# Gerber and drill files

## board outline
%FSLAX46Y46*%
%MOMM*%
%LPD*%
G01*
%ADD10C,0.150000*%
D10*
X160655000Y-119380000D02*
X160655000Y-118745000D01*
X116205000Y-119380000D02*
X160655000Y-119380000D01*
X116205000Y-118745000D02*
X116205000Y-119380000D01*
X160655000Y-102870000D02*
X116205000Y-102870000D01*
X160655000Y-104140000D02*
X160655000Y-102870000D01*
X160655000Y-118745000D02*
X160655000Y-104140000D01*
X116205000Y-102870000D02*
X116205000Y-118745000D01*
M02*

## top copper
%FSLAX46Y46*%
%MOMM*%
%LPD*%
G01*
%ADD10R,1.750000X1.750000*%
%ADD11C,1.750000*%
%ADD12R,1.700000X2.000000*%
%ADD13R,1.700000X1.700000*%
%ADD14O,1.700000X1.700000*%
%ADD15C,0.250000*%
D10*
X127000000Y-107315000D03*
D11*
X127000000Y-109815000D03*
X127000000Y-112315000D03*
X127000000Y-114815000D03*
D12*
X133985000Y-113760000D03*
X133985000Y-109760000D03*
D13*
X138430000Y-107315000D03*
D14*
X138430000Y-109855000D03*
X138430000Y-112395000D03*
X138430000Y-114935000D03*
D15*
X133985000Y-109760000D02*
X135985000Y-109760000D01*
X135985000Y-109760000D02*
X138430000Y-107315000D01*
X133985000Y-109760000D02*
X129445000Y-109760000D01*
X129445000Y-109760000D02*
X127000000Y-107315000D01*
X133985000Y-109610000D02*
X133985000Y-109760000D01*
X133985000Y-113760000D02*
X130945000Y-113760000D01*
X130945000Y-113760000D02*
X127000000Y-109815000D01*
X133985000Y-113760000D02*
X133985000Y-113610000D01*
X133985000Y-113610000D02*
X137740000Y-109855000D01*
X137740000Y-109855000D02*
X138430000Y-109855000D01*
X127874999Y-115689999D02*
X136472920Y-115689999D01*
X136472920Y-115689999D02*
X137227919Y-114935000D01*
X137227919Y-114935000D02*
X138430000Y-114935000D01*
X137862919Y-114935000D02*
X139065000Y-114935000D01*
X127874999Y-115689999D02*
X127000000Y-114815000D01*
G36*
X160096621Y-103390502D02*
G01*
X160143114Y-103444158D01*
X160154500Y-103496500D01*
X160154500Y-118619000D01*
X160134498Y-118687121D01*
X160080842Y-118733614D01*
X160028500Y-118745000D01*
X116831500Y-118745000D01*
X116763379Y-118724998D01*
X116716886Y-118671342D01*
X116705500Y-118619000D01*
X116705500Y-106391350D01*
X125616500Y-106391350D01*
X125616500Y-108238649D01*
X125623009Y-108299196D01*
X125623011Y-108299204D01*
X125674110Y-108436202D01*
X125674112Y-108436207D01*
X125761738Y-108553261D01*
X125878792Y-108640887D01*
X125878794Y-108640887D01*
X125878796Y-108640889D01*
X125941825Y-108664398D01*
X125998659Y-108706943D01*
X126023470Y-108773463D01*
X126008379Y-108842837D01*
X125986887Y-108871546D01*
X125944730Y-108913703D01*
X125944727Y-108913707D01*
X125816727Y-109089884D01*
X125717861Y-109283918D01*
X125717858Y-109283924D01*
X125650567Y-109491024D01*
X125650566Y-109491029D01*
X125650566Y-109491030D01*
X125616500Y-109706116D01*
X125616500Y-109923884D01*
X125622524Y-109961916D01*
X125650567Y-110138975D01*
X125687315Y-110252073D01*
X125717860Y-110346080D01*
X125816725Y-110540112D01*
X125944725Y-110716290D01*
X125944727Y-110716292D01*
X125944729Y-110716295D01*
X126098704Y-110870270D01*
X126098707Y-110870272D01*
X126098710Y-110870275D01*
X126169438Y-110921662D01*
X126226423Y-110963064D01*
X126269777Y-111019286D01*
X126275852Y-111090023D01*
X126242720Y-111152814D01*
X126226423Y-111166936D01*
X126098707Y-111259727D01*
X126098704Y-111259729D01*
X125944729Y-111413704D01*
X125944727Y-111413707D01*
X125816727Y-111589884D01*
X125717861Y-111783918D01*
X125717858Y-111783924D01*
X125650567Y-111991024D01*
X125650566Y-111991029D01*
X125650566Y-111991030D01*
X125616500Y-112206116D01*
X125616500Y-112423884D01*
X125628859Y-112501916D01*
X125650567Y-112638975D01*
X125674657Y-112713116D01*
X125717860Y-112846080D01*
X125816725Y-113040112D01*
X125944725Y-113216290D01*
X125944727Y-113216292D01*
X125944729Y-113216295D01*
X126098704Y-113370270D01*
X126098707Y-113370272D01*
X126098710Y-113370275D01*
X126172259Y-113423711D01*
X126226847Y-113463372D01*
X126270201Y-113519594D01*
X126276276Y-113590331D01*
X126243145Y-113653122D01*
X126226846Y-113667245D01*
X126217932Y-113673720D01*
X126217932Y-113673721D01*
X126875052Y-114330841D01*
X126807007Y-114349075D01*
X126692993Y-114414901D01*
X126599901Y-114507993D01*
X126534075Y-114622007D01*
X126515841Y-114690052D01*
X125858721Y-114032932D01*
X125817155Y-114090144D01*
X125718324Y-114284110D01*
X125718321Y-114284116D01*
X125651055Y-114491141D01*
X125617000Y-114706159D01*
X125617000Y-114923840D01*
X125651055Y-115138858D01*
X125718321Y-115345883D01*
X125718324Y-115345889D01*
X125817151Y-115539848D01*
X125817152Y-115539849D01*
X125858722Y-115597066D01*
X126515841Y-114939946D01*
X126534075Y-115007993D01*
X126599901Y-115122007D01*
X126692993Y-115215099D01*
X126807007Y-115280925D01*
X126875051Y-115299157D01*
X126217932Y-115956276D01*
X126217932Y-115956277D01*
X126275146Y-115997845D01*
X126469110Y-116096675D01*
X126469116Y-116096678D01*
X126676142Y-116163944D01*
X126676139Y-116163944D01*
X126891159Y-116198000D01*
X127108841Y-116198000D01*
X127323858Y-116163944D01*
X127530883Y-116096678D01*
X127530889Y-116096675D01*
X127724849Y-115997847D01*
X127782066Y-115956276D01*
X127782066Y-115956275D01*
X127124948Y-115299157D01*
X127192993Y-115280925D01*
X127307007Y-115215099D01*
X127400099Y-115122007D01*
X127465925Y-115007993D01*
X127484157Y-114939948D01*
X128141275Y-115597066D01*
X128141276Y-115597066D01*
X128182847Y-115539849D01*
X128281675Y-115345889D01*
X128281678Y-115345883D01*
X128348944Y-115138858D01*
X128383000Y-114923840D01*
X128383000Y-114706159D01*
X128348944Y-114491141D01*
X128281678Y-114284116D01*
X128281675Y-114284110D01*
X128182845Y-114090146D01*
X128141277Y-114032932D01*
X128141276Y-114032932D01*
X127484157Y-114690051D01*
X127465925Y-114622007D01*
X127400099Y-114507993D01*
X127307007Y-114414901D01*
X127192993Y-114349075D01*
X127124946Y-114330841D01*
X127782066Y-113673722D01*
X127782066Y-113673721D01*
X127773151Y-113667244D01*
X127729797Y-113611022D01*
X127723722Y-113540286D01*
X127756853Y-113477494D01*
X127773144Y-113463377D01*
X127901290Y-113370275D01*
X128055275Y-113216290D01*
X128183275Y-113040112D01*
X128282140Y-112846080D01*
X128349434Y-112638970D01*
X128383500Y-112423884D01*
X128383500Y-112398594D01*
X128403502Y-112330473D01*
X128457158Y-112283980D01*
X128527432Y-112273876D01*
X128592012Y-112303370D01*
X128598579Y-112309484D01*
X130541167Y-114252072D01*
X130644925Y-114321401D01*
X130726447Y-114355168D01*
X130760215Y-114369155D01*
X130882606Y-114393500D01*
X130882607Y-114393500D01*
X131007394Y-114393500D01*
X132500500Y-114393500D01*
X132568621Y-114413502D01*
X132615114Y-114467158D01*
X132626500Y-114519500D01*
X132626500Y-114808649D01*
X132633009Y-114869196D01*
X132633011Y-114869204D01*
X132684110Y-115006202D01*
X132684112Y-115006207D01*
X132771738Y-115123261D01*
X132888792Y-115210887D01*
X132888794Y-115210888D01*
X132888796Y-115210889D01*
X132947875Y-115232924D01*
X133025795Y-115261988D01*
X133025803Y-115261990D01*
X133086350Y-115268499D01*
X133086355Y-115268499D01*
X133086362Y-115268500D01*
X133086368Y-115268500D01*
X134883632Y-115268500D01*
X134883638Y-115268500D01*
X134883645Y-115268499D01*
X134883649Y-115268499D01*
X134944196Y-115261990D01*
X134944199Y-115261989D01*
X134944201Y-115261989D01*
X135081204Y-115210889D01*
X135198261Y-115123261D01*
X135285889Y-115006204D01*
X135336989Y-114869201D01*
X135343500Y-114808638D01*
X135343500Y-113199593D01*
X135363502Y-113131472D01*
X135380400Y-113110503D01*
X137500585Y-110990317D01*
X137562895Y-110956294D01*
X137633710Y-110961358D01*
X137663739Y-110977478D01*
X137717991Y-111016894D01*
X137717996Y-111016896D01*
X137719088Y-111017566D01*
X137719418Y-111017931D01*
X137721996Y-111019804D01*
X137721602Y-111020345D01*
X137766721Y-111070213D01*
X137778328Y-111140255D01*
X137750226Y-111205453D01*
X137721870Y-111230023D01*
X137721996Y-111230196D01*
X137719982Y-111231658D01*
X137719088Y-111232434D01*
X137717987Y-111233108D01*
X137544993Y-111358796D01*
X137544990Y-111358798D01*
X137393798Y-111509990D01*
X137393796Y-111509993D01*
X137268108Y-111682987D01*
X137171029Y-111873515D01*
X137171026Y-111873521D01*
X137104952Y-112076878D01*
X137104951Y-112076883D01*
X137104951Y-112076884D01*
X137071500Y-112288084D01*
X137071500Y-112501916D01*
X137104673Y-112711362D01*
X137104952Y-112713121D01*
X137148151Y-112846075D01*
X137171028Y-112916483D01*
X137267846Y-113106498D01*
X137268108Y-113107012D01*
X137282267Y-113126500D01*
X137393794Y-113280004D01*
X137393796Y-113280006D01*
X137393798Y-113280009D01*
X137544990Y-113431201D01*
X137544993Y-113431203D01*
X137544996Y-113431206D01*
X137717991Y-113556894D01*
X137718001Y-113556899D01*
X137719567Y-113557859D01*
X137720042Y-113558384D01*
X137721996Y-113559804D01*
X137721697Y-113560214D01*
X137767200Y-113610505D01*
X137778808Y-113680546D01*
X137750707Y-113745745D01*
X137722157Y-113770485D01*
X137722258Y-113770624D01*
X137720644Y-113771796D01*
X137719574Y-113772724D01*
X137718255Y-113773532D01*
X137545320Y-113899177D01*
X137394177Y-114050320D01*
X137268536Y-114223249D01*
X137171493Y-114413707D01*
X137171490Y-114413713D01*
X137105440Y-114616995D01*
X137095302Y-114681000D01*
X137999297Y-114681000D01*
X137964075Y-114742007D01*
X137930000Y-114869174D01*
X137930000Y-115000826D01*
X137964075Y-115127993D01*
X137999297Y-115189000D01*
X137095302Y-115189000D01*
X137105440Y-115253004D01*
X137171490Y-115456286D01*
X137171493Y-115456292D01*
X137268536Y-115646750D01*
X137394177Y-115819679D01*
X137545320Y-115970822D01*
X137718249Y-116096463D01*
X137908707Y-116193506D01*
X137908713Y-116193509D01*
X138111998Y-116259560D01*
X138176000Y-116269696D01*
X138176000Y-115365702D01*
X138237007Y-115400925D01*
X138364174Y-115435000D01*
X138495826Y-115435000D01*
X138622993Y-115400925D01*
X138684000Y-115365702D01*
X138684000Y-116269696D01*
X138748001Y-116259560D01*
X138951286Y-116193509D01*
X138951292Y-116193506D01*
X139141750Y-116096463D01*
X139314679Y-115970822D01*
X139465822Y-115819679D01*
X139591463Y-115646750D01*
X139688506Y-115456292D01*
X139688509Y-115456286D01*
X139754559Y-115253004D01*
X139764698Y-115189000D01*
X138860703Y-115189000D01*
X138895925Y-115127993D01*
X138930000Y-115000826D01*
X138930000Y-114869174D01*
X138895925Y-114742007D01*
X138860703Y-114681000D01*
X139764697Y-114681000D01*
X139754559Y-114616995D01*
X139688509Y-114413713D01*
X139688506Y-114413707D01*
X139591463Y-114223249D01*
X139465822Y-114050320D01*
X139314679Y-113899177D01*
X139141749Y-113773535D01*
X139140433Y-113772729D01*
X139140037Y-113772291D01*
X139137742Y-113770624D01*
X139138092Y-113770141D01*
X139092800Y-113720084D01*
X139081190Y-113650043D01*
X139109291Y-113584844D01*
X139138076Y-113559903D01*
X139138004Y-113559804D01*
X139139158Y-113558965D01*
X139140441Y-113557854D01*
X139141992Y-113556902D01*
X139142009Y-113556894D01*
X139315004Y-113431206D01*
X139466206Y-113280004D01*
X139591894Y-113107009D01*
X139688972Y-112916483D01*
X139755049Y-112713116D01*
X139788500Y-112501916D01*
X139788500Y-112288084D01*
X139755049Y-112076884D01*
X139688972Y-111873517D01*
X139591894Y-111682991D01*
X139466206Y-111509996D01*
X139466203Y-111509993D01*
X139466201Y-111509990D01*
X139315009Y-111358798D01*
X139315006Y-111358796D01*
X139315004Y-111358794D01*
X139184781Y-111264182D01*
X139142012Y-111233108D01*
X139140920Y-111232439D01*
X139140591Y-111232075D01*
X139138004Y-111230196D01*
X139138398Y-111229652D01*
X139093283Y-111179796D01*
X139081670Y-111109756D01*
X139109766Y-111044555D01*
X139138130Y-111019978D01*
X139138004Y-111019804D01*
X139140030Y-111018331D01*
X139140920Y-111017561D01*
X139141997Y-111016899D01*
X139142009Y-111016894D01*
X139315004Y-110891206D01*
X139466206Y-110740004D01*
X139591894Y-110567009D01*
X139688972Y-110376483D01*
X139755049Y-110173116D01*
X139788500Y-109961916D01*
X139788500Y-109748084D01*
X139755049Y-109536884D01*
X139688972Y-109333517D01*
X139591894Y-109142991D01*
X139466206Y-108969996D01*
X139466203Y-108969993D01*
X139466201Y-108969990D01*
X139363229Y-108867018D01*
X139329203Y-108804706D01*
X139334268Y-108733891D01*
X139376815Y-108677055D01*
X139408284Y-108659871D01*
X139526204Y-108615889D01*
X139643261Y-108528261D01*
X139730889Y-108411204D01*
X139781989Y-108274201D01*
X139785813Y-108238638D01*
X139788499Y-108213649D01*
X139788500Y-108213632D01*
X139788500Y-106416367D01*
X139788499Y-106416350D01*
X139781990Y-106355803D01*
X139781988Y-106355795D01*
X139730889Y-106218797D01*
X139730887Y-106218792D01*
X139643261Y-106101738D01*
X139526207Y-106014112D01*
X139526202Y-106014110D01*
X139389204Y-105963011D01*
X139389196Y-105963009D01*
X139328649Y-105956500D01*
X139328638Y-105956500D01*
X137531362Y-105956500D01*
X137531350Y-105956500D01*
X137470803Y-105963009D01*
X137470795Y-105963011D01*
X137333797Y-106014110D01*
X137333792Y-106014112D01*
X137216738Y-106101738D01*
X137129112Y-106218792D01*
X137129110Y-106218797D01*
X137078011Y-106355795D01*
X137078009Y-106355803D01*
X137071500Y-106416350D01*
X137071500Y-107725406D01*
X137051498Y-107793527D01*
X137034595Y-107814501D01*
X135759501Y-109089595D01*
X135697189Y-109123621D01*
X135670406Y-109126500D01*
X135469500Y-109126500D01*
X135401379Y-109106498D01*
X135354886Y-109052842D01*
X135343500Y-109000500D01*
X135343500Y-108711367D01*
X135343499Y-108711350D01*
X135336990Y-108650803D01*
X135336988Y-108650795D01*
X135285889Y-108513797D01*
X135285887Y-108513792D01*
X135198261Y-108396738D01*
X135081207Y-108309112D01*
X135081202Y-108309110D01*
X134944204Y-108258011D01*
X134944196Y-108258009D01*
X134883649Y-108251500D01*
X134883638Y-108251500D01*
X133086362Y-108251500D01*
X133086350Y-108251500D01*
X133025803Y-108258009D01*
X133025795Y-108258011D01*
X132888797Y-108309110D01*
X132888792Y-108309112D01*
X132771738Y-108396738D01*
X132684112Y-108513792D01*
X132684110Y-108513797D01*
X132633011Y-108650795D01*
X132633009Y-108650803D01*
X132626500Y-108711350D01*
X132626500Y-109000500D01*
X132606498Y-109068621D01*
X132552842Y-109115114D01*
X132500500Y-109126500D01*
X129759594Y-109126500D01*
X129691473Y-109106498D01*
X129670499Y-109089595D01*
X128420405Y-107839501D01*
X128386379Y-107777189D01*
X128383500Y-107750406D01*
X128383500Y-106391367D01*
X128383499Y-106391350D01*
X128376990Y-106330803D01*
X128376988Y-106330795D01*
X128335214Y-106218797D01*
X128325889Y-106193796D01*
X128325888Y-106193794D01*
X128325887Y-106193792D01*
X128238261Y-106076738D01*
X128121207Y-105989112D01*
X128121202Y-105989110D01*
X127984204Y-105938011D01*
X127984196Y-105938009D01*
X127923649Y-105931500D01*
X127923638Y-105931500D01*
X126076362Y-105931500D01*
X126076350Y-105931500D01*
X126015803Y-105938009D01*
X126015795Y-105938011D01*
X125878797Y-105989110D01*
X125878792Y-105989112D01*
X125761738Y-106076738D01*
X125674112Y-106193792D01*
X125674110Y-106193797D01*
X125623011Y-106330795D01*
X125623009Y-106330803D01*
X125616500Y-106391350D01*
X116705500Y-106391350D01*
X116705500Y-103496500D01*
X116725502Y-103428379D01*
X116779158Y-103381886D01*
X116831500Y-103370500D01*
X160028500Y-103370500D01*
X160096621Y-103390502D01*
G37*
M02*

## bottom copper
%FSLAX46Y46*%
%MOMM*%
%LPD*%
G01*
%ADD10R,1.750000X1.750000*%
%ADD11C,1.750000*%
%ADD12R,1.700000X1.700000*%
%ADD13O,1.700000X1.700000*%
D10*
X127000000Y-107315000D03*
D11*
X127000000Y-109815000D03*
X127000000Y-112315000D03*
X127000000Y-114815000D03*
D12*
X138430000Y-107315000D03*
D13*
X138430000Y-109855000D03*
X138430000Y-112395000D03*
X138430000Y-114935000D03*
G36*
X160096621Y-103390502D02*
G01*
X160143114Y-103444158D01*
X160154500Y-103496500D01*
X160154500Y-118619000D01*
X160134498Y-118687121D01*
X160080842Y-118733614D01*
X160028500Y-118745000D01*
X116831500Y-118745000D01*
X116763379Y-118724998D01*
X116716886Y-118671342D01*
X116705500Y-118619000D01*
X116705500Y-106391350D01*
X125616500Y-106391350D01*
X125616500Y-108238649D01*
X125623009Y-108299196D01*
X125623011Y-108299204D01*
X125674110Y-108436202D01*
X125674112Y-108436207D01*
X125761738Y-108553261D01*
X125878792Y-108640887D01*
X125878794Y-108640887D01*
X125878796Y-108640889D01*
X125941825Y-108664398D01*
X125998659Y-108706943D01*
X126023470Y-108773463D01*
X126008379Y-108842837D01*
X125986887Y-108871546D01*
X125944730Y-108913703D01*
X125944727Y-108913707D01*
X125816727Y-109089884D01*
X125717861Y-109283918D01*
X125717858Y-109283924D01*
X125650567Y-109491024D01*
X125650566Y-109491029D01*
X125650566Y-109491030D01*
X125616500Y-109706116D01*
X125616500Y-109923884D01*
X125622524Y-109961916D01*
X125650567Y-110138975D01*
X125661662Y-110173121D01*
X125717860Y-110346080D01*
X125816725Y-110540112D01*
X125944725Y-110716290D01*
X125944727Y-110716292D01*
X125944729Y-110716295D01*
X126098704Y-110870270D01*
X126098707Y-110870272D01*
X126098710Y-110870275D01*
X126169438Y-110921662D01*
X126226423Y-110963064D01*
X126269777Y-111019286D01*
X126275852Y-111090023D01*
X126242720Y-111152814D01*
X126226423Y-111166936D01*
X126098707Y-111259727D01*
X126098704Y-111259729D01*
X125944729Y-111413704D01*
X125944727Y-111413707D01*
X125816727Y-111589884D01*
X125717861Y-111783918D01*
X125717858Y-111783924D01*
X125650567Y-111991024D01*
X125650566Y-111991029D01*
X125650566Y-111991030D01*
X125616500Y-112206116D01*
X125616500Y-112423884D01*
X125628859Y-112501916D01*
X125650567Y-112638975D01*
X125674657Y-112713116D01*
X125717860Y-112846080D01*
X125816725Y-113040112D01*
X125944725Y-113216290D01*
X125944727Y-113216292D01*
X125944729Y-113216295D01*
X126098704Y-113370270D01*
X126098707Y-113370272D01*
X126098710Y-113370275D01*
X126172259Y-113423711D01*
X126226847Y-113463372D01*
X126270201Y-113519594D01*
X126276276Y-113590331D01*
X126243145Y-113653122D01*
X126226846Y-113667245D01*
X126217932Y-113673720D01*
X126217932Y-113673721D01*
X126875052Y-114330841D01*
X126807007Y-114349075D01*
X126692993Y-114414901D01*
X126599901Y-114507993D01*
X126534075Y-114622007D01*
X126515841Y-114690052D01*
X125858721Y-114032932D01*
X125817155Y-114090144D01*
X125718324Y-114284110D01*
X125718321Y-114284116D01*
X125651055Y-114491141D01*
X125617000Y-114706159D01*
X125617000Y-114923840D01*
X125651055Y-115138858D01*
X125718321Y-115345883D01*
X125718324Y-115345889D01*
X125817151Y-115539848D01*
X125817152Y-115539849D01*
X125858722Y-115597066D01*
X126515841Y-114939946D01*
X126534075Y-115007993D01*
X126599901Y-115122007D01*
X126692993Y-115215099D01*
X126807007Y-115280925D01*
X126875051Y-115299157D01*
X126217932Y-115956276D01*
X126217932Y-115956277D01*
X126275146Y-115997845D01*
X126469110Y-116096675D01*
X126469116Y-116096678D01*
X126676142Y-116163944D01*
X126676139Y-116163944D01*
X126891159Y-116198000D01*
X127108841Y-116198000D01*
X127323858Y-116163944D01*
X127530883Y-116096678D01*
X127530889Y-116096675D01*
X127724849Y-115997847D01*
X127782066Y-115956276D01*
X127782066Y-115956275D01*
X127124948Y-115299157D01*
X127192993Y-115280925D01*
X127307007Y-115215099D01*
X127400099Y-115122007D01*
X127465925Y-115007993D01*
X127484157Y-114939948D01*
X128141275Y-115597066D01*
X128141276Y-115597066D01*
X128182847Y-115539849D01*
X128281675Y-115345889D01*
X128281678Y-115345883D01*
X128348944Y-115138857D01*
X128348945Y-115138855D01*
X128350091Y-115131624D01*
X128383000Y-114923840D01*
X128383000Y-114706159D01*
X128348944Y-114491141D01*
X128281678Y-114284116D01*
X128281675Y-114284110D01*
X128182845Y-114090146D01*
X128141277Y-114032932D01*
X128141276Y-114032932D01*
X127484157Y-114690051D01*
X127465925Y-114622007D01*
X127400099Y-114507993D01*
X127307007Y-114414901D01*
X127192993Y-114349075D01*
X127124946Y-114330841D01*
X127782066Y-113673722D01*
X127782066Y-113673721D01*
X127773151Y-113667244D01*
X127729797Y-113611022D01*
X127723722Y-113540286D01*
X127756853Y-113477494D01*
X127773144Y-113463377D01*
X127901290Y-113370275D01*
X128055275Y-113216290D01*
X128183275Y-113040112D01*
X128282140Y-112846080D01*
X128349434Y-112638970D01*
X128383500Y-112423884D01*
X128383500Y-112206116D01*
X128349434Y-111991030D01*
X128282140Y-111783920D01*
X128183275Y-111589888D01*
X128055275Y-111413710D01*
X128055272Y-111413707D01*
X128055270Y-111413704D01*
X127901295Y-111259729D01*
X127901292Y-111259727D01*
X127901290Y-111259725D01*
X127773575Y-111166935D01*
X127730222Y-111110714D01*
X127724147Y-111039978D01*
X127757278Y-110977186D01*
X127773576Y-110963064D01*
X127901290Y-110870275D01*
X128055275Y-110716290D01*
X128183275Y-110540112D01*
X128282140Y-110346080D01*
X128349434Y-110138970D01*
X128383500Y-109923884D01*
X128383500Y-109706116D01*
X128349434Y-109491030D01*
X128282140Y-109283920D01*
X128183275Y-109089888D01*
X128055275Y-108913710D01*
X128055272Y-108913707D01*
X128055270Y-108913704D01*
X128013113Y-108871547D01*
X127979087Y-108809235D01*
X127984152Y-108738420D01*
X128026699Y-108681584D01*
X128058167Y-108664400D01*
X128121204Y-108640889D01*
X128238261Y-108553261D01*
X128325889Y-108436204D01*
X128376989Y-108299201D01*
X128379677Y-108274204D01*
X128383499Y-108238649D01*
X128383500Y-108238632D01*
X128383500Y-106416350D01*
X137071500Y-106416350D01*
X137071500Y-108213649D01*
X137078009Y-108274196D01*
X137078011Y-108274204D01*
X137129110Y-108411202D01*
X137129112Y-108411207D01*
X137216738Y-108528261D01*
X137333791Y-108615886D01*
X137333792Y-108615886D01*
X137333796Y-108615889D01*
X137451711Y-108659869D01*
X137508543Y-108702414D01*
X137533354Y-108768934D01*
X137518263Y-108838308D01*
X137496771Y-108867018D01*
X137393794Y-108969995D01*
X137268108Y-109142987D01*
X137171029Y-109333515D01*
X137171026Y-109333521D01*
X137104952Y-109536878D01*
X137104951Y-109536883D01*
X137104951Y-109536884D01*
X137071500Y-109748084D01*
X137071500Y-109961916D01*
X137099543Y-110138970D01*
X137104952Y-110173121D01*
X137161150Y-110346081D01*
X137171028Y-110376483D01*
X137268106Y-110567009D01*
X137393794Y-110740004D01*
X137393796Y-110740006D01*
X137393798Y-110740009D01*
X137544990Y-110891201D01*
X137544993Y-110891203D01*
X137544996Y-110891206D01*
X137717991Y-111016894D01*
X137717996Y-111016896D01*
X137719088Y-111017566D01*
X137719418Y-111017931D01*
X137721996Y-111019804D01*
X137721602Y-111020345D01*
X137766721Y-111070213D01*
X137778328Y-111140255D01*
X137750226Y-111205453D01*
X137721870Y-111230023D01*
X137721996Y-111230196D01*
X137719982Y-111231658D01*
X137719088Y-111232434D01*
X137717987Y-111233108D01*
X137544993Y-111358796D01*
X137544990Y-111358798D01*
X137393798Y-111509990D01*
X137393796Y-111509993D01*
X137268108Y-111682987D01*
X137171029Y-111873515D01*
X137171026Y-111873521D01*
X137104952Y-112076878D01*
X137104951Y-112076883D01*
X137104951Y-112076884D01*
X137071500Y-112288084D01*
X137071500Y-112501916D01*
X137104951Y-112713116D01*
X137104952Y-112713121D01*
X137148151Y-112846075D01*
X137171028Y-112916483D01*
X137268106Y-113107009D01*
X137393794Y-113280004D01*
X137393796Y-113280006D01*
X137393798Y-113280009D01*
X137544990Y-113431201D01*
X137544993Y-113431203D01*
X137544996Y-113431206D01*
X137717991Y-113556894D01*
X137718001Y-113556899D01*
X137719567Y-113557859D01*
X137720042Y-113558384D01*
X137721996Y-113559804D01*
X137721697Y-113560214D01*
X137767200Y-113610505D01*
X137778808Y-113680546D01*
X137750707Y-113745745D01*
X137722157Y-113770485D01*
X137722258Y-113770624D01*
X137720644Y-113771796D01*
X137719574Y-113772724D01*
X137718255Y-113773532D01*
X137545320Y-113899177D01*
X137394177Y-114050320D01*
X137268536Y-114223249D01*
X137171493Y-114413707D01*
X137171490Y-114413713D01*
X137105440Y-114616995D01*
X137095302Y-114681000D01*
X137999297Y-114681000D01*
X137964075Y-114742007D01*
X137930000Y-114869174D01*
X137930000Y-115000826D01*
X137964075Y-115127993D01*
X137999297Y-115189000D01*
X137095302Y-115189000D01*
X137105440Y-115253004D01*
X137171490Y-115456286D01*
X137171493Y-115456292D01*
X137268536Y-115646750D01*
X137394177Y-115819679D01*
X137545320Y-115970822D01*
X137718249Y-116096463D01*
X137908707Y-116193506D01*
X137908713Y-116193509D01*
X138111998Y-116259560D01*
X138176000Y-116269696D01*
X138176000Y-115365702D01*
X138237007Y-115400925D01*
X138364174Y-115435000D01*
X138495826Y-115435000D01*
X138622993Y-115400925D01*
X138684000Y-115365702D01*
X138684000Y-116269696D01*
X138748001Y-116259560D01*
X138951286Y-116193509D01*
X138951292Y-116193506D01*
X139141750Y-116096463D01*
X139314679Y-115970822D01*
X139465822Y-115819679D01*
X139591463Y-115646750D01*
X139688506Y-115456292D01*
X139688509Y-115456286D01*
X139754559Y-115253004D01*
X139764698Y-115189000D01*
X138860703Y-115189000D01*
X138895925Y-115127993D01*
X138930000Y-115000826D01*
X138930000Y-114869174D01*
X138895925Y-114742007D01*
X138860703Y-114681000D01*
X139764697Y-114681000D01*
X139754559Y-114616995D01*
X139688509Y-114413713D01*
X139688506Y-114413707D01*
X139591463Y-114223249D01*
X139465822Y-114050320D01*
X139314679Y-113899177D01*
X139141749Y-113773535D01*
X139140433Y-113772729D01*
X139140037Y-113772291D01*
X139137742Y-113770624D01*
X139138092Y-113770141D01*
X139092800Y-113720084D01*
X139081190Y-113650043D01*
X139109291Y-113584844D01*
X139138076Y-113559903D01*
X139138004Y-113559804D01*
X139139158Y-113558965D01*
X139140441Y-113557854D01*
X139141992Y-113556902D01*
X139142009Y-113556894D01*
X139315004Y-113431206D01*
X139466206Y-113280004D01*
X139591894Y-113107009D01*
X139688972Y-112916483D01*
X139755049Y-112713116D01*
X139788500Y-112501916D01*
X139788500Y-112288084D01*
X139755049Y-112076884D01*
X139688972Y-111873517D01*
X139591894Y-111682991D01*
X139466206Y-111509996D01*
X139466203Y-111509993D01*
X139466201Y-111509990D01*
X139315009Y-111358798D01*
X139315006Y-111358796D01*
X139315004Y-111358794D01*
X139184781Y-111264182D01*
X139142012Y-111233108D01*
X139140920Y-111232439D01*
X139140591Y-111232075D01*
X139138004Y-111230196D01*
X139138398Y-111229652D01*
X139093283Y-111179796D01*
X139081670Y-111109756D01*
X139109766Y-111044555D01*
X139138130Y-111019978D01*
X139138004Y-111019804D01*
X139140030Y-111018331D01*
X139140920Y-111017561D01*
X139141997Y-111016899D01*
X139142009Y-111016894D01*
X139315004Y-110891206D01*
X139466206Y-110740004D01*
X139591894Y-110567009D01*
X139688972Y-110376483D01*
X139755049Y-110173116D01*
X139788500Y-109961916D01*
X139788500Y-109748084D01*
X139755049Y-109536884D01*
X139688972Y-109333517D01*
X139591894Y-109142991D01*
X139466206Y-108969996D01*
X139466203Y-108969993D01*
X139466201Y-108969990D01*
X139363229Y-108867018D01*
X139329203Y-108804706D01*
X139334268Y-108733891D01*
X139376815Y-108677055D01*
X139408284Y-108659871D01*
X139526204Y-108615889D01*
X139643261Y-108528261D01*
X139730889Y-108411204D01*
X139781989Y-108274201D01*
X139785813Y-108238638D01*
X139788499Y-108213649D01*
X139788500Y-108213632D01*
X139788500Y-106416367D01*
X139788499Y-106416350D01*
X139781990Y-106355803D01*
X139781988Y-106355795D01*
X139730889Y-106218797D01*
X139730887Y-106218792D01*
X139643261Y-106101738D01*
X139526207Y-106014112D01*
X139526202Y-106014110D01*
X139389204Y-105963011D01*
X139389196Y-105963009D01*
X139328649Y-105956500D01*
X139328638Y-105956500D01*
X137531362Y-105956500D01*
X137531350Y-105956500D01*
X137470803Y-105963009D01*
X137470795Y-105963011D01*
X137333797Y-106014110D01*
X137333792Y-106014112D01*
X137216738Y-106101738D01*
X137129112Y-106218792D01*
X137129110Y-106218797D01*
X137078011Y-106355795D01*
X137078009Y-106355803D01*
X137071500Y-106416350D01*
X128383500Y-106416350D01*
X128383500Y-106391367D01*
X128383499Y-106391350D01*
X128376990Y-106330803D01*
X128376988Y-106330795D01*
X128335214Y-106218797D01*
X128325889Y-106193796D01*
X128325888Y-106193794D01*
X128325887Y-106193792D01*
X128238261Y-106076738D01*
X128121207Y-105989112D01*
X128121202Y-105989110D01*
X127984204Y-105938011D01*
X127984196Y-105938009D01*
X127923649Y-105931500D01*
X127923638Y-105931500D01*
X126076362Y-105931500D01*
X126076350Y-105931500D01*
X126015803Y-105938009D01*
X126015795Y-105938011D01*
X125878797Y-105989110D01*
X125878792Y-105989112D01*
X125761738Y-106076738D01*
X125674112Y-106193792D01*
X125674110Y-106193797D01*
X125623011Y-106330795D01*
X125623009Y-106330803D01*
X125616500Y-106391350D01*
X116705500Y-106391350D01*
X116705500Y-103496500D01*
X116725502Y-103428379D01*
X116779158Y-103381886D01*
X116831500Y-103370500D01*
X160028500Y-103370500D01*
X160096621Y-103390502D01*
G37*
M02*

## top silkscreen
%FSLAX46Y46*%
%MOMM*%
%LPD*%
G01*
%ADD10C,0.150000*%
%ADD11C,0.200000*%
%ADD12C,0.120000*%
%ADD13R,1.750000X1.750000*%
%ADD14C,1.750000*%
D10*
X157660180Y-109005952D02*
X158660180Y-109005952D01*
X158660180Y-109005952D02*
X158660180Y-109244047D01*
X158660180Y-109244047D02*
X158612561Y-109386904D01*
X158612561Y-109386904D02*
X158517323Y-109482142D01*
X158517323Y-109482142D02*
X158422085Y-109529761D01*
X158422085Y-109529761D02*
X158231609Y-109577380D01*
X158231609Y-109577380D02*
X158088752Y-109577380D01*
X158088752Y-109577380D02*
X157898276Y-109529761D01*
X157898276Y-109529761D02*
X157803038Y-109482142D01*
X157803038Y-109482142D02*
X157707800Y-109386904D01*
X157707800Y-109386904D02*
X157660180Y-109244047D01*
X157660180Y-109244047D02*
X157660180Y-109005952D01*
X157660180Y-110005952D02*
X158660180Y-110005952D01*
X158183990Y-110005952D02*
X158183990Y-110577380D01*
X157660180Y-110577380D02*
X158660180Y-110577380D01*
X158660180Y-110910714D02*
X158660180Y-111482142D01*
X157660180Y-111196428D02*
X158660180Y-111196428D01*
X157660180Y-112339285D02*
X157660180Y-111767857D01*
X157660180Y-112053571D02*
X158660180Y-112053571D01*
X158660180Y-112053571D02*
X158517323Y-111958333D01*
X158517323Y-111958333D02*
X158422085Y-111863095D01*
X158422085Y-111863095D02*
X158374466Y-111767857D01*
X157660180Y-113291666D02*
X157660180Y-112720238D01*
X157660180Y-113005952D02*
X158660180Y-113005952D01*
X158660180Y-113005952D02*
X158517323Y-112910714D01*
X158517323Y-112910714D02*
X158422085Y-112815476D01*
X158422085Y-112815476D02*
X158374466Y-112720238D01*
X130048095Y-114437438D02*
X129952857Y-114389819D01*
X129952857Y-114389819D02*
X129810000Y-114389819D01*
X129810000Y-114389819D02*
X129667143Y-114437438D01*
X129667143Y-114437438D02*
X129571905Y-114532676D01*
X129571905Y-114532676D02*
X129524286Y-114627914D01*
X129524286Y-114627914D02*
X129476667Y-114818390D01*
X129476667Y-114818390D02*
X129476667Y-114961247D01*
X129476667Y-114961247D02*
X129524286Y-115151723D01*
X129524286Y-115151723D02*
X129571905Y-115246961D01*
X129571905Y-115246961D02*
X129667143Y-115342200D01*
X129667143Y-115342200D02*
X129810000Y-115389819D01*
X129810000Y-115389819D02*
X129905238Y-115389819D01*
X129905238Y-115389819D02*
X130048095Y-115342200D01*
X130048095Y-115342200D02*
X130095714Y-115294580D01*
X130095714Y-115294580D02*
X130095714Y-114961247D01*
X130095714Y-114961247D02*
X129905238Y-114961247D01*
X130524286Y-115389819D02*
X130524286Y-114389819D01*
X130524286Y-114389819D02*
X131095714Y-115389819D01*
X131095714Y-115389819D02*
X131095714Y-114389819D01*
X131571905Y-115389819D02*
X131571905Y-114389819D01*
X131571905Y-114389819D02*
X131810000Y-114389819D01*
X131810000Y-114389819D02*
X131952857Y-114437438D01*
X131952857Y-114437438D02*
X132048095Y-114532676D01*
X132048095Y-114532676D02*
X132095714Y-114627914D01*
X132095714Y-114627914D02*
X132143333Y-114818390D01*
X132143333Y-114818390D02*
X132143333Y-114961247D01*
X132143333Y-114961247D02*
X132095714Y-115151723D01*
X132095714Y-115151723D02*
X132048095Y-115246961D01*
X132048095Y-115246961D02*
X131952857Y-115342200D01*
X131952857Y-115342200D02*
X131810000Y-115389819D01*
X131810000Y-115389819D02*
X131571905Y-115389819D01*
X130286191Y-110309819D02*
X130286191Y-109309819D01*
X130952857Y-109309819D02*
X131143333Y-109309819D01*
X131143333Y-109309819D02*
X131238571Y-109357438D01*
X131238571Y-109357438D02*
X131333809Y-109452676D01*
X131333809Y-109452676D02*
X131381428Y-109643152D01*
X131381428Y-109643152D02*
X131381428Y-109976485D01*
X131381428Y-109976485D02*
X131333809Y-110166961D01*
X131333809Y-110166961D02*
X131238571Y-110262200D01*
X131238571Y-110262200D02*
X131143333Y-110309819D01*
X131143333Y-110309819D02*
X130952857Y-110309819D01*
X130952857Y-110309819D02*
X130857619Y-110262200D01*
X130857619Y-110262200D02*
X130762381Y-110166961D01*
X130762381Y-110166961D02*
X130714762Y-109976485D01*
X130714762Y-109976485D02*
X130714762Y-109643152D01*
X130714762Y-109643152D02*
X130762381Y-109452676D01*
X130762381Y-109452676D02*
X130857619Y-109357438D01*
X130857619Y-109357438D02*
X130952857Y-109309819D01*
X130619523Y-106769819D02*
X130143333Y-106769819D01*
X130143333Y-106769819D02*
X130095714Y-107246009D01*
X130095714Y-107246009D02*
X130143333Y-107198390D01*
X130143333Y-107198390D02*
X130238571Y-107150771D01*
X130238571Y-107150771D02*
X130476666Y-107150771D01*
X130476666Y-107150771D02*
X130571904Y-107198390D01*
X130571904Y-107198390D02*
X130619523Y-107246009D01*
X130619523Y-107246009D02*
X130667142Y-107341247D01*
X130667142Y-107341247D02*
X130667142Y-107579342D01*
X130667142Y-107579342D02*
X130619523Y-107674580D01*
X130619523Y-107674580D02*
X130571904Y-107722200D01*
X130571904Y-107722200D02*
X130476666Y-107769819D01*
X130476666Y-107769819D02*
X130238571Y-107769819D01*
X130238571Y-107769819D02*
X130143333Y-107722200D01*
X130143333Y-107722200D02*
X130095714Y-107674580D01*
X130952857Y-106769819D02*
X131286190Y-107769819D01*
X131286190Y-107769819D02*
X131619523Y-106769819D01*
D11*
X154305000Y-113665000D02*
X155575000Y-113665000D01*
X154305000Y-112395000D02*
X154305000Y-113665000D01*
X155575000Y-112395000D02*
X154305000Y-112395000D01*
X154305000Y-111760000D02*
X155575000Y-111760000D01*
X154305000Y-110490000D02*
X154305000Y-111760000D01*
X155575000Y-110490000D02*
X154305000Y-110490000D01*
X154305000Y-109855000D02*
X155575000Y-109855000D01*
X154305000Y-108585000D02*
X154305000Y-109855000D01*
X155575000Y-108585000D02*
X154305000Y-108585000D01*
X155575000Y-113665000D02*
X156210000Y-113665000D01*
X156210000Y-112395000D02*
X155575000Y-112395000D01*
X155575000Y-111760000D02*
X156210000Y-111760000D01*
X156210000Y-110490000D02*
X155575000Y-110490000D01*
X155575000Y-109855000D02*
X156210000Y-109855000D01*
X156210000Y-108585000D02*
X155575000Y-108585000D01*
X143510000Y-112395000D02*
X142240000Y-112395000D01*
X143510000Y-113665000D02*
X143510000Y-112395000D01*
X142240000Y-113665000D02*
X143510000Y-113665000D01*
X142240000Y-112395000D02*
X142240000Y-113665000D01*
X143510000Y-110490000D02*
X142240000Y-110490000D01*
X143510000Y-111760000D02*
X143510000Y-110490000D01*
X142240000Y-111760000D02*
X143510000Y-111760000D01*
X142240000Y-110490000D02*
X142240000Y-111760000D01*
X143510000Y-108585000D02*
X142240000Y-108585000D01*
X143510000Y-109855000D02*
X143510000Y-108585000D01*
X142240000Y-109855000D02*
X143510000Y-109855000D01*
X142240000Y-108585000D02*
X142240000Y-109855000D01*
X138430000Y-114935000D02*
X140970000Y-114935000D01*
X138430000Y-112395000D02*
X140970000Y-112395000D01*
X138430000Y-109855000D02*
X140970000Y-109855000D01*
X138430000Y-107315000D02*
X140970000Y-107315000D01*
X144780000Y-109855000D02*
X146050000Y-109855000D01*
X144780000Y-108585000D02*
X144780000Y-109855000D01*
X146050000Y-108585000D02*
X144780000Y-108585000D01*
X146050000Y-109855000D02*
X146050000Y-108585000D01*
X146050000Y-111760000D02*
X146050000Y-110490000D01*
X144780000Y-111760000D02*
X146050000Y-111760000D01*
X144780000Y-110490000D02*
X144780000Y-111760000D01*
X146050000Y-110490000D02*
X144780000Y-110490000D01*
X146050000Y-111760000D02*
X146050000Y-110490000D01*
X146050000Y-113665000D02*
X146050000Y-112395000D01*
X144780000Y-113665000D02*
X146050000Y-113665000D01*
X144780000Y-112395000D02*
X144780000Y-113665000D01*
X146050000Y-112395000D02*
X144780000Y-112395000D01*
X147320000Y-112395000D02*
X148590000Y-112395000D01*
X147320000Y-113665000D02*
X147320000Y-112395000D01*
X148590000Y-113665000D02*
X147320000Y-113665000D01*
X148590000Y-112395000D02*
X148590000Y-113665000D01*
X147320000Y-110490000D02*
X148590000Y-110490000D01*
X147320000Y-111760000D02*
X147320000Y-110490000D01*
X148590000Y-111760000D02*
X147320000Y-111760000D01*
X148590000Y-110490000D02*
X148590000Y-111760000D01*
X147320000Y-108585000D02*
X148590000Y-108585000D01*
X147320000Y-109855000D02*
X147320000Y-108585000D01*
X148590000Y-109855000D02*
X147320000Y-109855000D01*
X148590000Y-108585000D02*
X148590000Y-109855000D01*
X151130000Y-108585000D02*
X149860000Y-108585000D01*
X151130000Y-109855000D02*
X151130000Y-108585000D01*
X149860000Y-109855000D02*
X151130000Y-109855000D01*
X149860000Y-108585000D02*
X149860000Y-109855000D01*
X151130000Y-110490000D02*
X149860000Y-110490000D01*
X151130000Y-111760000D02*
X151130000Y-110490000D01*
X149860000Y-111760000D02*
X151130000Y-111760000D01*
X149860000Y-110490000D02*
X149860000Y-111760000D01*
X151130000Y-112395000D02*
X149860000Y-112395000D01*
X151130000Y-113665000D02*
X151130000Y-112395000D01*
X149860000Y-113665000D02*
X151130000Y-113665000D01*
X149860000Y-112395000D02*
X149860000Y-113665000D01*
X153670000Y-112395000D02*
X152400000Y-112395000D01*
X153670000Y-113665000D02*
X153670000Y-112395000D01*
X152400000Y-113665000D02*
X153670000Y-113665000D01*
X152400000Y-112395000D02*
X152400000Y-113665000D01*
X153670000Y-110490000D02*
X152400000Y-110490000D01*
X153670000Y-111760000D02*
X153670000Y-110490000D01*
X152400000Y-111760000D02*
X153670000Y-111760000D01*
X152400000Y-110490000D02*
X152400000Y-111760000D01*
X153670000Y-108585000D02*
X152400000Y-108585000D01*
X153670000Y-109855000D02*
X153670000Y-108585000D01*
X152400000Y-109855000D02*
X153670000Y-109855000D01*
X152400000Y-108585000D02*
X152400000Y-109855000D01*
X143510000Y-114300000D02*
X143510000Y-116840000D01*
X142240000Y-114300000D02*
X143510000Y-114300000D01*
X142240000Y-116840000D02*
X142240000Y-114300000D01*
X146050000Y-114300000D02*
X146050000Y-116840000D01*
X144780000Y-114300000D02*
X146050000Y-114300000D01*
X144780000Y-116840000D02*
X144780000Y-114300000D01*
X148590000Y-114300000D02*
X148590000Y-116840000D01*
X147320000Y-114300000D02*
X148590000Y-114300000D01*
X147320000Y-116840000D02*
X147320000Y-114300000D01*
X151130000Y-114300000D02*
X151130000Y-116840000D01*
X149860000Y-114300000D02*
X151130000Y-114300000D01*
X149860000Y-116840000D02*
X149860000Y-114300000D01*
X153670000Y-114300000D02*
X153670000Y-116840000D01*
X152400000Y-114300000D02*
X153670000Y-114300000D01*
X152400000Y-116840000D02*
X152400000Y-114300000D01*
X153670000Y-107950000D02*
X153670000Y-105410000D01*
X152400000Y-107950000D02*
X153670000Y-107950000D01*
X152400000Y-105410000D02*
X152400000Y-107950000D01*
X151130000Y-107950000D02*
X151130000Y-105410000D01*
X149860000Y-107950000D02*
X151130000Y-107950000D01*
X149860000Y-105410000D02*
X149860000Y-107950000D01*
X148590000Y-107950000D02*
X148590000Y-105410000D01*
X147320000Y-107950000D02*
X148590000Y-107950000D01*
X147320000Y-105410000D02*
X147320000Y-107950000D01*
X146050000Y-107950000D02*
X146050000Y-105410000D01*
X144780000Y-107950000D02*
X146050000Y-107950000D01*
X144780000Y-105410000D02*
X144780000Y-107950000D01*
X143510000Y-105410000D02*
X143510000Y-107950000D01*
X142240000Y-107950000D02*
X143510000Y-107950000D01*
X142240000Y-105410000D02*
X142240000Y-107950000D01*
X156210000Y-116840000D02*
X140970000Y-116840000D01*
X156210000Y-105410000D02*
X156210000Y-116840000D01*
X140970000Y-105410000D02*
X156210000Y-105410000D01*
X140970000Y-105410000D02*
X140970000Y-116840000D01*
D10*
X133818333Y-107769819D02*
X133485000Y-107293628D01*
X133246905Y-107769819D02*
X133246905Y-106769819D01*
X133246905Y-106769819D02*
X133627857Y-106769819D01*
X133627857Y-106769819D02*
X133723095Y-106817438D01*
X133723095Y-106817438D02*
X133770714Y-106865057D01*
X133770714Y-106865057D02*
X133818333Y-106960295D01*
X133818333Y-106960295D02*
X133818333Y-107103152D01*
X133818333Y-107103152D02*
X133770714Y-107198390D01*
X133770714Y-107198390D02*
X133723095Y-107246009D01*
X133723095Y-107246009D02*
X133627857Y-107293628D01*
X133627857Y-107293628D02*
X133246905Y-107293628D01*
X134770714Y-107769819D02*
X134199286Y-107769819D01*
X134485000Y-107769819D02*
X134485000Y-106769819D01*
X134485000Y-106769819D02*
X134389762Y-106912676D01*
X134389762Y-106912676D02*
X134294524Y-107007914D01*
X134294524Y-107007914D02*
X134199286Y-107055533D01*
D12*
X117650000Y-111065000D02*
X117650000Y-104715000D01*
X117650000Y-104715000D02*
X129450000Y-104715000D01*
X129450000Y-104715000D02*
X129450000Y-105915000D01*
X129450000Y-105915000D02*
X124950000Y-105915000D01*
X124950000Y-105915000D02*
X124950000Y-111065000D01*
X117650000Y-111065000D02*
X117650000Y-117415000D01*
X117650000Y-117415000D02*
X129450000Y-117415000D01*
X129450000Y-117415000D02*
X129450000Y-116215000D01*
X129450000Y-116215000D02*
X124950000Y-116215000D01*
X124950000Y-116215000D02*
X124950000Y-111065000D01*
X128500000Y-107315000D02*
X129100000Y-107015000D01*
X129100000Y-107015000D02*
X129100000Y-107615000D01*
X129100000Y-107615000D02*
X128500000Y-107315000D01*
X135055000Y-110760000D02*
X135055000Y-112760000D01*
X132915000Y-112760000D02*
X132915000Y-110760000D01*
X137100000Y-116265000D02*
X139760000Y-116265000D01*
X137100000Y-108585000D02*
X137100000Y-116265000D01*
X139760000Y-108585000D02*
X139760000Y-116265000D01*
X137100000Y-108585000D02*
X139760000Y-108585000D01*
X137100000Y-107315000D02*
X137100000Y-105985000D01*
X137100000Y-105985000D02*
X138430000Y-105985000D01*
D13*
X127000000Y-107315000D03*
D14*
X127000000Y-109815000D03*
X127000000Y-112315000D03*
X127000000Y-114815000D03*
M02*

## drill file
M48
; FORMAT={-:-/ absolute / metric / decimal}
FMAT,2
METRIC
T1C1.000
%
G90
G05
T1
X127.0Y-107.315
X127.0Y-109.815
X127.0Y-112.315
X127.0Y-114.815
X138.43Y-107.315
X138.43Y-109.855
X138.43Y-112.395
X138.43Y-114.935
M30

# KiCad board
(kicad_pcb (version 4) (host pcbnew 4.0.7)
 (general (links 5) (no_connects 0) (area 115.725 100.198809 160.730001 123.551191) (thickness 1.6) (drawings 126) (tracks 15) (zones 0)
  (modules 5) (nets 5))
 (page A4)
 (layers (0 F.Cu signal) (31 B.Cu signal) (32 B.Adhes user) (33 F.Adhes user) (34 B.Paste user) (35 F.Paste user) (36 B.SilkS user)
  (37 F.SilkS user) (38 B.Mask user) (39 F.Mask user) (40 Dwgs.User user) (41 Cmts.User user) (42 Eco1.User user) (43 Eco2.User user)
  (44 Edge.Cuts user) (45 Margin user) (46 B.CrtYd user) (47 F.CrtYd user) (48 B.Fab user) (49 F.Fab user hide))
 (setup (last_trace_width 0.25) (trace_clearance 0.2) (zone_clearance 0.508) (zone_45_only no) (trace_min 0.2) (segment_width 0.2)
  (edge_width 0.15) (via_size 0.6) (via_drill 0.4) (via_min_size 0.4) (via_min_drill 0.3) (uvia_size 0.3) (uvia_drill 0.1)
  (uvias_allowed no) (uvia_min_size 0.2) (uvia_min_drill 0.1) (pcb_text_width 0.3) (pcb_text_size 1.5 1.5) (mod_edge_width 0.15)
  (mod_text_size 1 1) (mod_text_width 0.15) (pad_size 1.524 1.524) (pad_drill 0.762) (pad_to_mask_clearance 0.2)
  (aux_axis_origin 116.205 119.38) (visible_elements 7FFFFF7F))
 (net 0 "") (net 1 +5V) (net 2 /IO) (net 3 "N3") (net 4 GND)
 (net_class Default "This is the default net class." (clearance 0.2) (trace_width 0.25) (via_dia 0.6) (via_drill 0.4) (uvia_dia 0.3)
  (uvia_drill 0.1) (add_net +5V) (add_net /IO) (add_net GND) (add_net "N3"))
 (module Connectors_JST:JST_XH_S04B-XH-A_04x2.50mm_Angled (layer F.Cu) (at 127 107.315 270)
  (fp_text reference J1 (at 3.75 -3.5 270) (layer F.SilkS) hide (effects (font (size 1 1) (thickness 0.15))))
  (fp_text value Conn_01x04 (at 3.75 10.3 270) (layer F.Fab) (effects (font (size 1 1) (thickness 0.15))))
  (fp_line (start 3.75 9.35) (end -2.6 9.35) (layer F.SilkS) (width 0.12))
  (fp_line (start -2.6 9.35) (end -2.6 -2.45) (layer F.SilkS) (width 0.12))
  (fp_line (start -2.6 -2.45) (end -1.4 -2.45) (layer F.SilkS) (width 0.12))
  (fp_line (start -1.4 -2.45) (end -1.4 2.05) (layer F.SilkS) (width 0.12))
  (fp_line (start -1.4 2.05) (end 3.75 2.05) (layer F.SilkS) (width 0.12))
  (fp_line (start 3.75 9.35) (end 10.1 9.35) (layer F.SilkS) (width 0.12))
  (fp_line (start 10.1 9.35) (end 10.1 -2.45) (layer F.SilkS) (width 0.12))
  (fp_line (start 10.1 -2.45) (end 8.9 -2.45) (layer F.SilkS) (width 0.12))
  (fp_line (start 8.9 -2.45) (end 8.9 2.05) (layer F.SilkS) (width 0.12))
  (fp_line (start 8.9 2.05) (end 3.75 2.05) (layer F.SilkS) (width 0.12))
  (fp_line (start 0 -1.5) (end -0.3 -2.1) (layer F.SilkS) (width 0.12))
  (fp_line (start -0.3 -2.1) (end 0.3 -2.1) (layer F.SilkS) (width 0.12))
  (fp_line (start 0.3 -2.1) (end 0 -1.5) (layer F.SilkS) (width 0.12))
  (pad 1 thru_hole rect (at 0 0 270) (size 1.75 1.75) (drill 1) (layers *.Cu *.Mask F.SilkS) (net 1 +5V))
  (pad 2 thru_hole circle (at 2.5 0 270) (size 1.75 1.75) (drill 1) (layers *.Cu *.Mask F.SilkS) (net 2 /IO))
  (pad 3 thru_hole circle (at 5 0 270) (size 1.75 1.75) (drill 1) (layers *.Cu *.Mask F.SilkS) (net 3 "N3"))
  (pad 4 thru_hole circle (at 7.5 0 270) (size 1.75 1.75) (drill 1) (layers *.Cu *.Mask F.SilkS) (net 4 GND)))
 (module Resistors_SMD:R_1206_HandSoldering (layer F.Cu) (at 133.985 111.76 90)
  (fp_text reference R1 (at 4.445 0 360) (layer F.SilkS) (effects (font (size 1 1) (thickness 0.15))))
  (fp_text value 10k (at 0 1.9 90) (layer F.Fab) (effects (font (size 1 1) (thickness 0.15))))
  (fp_line (start 1 1.07) (end -1 1.07) (layer F.SilkS) (width 0.12))
  (fp_line (start -1 -1.07) (end 1 -1.07) (layer F.SilkS) (width 0.12))
  (pad 1 smd rect (at -2 0 90) (size 2 1.7) (layers F.Cu F.Paste F.Mask) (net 2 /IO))
  (pad 2 smd rect (at 2 0 90) (size 2 1.7) (layers F.Cu F.Paste F.Mask) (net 1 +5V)))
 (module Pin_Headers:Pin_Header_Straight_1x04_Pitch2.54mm (layer F.Cu) (at 138.43 107.315)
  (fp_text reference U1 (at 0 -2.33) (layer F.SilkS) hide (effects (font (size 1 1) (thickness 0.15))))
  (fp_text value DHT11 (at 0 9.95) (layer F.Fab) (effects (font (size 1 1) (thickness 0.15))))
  (fp_line (start -1.33 8.95) (end 1.33 8.95) (layer F.SilkS) (width 0.12))
  (fp_line (start -1.33 1.27) (end -1.33 8.95) (layer F.SilkS) (width 0.12))
  (fp_line (start 1.33 1.27) (end 1.33 8.95) (layer F.SilkS) (width 0.12))
  (fp_line (start -1.33 1.27) (end 1.33 1.27) (layer F.SilkS) (width 0.12))
  (fp_line (start -1.33 0) (end -1.33 -1.33) (layer F.SilkS) (width 0.12))
  (fp_line (start -1.33 -1.33) (end 0 -1.33) (layer F.SilkS) (width 0.12))
  (pad 1 thru_hole rect (at 0 0) (size 1.7 1.7) (drill 1) (layers *.Cu *.Mask) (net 1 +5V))
  (pad 2 thru_hole oval (at 0 2.54) (size 1.7 1.7) (drill 1) (layers *.Cu *.Mask) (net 2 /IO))
  (pad 3 thru_hole oval (at 0 5.08) (size 1.7 1.7) (drill 1) (layers *.Cu *.Mask))
  (pad 4 thru_hole oval (at 0 7.62) (size 1.7 1.7) (drill 1) (layers *.Cu *.Mask) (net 4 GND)))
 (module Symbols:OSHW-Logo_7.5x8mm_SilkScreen (layer B.Cu) (at 132.715 111.125)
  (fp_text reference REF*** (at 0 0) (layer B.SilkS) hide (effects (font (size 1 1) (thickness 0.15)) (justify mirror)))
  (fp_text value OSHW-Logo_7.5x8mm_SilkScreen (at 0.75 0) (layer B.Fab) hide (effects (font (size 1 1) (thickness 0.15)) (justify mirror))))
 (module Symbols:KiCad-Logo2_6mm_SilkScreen (layer B.Cu) (at 121.285 111.125 270)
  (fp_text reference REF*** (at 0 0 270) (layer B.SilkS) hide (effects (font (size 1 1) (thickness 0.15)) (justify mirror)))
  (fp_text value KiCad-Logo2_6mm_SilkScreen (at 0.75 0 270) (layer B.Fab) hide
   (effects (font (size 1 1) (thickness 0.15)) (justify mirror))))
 (gr_line (start 160.655 119.38) (end 160.655 118.745) (layer Edge.Cuts) (width 0.15))
 (gr_line (start 116.205 119.38) (end 160.655 119.38) (layer Edge.Cuts) (width 0.15))
 (gr_line (start 116.205 118.745) (end 116.205 119.38) (layer Edge.Cuts) (width 0.15))
 (gr_line (start 160.655 102.87) (end 116.205 102.87) (layer Edge.Cuts) (width 0.15))
 (gr_line (start 160.655 104.14) (end 160.655 102.87) (layer Edge.Cuts) (width 0.15))
 (gr_line (start 160.655 118.745) (end 160.655 104.14) (layer Edge.Cuts) (width 0.15))
 (gr_line (start 116.205 102.87) (end 116.205 118.745) (layer Edge.Cuts) (width 0.15))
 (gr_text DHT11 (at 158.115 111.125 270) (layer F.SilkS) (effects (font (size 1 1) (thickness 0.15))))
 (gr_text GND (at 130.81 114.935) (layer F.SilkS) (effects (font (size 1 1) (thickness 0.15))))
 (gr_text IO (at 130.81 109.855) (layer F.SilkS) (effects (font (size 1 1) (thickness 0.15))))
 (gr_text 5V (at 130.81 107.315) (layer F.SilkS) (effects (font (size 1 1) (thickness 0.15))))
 (gr_line (start 154.305 113.665) (end 155.575 113.665) (layer F.SilkS) (width 0.2))
 (gr_line (start 154.305 112.395) (end 154.305 113.665) (layer F.SilkS) (width 0.2))
 (gr_line (start 155.575 112.395) (end 154.305 112.395) (layer F.SilkS) (width 0.2))
 (gr_line (start 154.305 111.76) (end 155.575 111.76) (layer F.SilkS) (width 0.2))
 (gr_line (start 154.305 110.49) (end 154.305 111.76) (layer F.SilkS) (width 0.2))
 (gr_line (start 155.575 110.49) (end 154.305 110.49) (layer F.SilkS) (width 0.2))
 (gr_line (start 154.305 109.855) (end 155.575 109.855) (layer F.SilkS) (width 0.2))
 (gr_line (start 154.305 108.585) (end 154.305 109.855) (layer F.SilkS) (width 0.2))
 (gr_line (start 155.575 108.585) (end 154.305 108.585) (layer F.SilkS) (width 0.2))
 (gr_line (start 155.575 113.665) (end 156.21 113.665) (layer F.SilkS) (width 0.2))
 (gr_line (start 156.21 112.395) (end 155.575 112.395) (layer F.SilkS) (width 0.2))
 (gr_line (start 155.575 111.76) (end 156.21 111.76) (layer F.SilkS) (width 0.2))
 (gr_line (start 156.21 110.49) (end 155.575 110.49) (layer F.SilkS) (width 0.2))
 (gr_line (start 155.575 109.855) (end 156.21 109.855) (layer F.SilkS) (width 0.2))
 (gr_line (start 156.21 108.585) (end 155.575 108.585) (layer F.SilkS) (width 0.2))
 (gr_line (start 143.51 112.395) (end 142.24 112.395) (layer F.SilkS) (width 0.2))
 (gr_line (start 143.51 113.665) (end 143.51 112.395) (layer F.SilkS) (width 0.2))
 (gr_line (start 142.24 113.665) (end 143.51 113.665) (layer F.SilkS) (width 0.2))
 (gr_line (start 142.24 112.395) (end 142.24 113.665) (layer F.SilkS) (width 0.2))
 (gr_line (start 143.51 110.49) (end 142.24 110.49) (layer F.SilkS) (width 0.2))
 (gr_line (start 143.51 111.76) (end 143.51 110.49) (layer F.SilkS) (width 0.2))
 (gr_line (start 142.24 111.76) (end 143.51 111.76) (layer F.SilkS) (width 0.2))
 (gr_line (start 142.24 110.49) (end 142.24 111.76) (layer F.SilkS) (width 0.2))
 (gr_line (start 143.51 108.585) (end 142.24 108.585) (layer F.SilkS) (width 0.2))
 (gr_line (start 143.51 109.855) (end 143.51 108.585) (layer F.SilkS) (width 0.2))
 (gr_line (start 142.24 109.855) (end 143.51 109.855) (layer F.SilkS) (width 0.2))
 (gr_line (start 142.24 108.585) (end 142.24 109.855) (layer F.SilkS) (width 0.2))
 (gr_line (start 138.43 114.935) (end 140.97 114.935) (layer F.SilkS) (width 0.2))
 (gr_line (start 138.43 112.395) (end 140.97 112.395) (layer F.SilkS) (width 0.2))
 (gr_line (start 138.43 109.855) (end 140.97 109.855) (layer F.SilkS) (width 0.2))
 (gr_line (start 138.43 107.315) (end 140.97 107.315) (layer F.SilkS) (width 0.2))
 (gr_line (start 144.78 109.855) (end 146.05 109.855) (layer F.SilkS) (width 0.2))
 (gr_line (start 144.78 108.585) (end 144.78 109.855) (layer F.SilkS) (width 0.2))
 (gr_line (start 146.05 108.585) (end 144.78 108.585) (layer F.SilkS) (width 0.2))
 (gr_line (start 146.05 109.855) (end 146.05 108.585) (layer F.SilkS) (width 0.2))
 (gr_line (start 146.05 111.76) (end 146.05 110.49) (layer F.SilkS) (width 0.2))
 (gr_line (start 144.78 111.76) (end 146.05 111.76) (layer F.SilkS) (width 0.2))
 (gr_line (start 144.78 110.49) (end 144.78 111.76) (layer F.SilkS) (width 0.2))
 (gr_line (start 146.05 110.49) (end 144.78 110.49) (layer F.SilkS) (width 0.2))
 (gr_line (start 146.05 111.76) (end 146.05 110.49) (layer F.SilkS) (width 0.2))
 (gr_line (start 146.05 113.665) (end 146.05 112.395) (layer F.SilkS) (width 0.2))
 (gr_line (start 144.78 113.665) (end 146.05 113.665) (layer F.SilkS) (width 0.2))
 (gr_line (start 144.78 112.395) (end 144.78 113.665) (layer F.SilkS) (width 0.2))
 (gr_line (start 146.05 112.395) (end 144.78 112.395) (layer F.SilkS) (width 0.2))
 (gr_line (start 147.32 112.395) (end 148.59 112.395) (layer F.SilkS) (width 0.2))
 (gr_line (start 147.32 113.665) (end 147.32 112.395) (layer F.SilkS) (width 0.2))
 (gr_line (start 148.59 113.665) (end 147.32 113.665) (layer F.SilkS) (width 0.2))
 (gr_line (start 148.59 112.395) (end 148.59 113.665) (layer F.SilkS) (width 0.2))
 (gr_line (start 147.32 110.49) (end 148.59 110.49) (layer F.SilkS) (width 0.2))
 (gr_line (start 147.32 111.76) (end 147.32 110.49) (layer F.SilkS) (width 0.2))
 (gr_line (start 148.59 111.76) (end 147.32 111.76) (layer F.SilkS) (width 0.2))
 (gr_line (start 148.59 110.49) (end 148.59 111.76) (layer F.SilkS) (width 0.2))
 (gr_line (start 147.32 108.585) (end 148.59 108.585) (layer F.SilkS) (width 0.2))
 (gr_line (start 147.32 109.855) (end 147.32 108.585) (layer F.SilkS) (width 0.2))
 (gr_line (start 148.59 109.855) (end 147.32 109.855) (layer F.SilkS) (width 0.2))
 (gr_line (start 148.59 108.585) (end 148.59 109.855) (layer F.SilkS) (width 0.2))
 (gr_line (start 151.13 108.585) (end 149.86 108.585) (layer F.SilkS) (width 0.2))
 (gr_line (start 151.13 109.855) (end 151.13 108.585) (layer F.SilkS) (width 0.2))
 (gr_line (start 149.86 109.855) (end 151.13 109.855) (layer F.SilkS) (width 0.2))
 (gr_line (start 149.86 108.585) (end 149.86 109.855) (layer F.SilkS) (width 0.2))
 (gr_line (start 151.13 110.49) (end 149.86 110.49) (layer F.SilkS) (width 0.2))
 (gr_line (start 151.13 111.76) (end 151.13 110.49) (layer F.SilkS) (width 0.2))
 (gr_line (start 149.86 111.76) (end 151.13 111.76) (layer F.SilkS) (width 0.2))
 (gr_line (start 149.86 110.49) (end 149.86 111.76) (layer F.SilkS) (width 0.2))
 (gr_line (start 151.13 112.395) (end 149.86 112.395) (layer F.SilkS) (width 0.2))
 (gr_line (start 151.13 113.665) (end 151.13 112.395) (layer F.SilkS) (width 0.2))
 (gr_line (start 149.86 113.665) (end 151.13 113.665) (layer F.SilkS) (width 0.2))
 (gr_line (start 149.86 112.395) (end 149.86 113.665) (layer F.SilkS) (width 0.2))
 (gr_line (start 153.67 112.395) (end 152.4 112.395) (layer F.SilkS) (width 0.2))
 (gr_line (start 153.67 113.665) (end 153.67 112.395) (layer F.SilkS) (width 0.2))
 (gr_line (start 152.4 113.665) (end 153.67 113.665) (layer F.SilkS) (width 0.2))
 (gr_line (start 152.4 112.395) (end 152.4 113.665) (layer F.SilkS) (width 0.2))
 (gr_line (start 153.67 110.49) (end 152.4 110.49) (layer F.SilkS) (width 0.2))
 (gr_line (start 153.67 111.76) (end 153.67 110.49) (layer F.SilkS) (width 0.2))
 (gr_line (start 152.4 111.76) (end 153.67 111.76) (layer F.SilkS) (width 0.2))
 (gr_line (start 152.4 110.49) (end 152.4 111.76) (layer F.SilkS) (width 0.2))
 (gr_line (start 153.67 108.585) (end 152.4 108.585) (layer F.SilkS) (width 0.2))
 (gr_line (start 153.67 109.855) (end 153.67 108.585) (layer F.SilkS) (width 0.2))
 (gr_line (start 152.4 109.855) (end 153.67 109.855) (layer F.SilkS) (width 0.2))
 (gr_line (start 152.4 108.585) (end 152.4 109.855) (layer F.SilkS) (width 0.2))
 (gr_line (start 143.51 114.3) (end 143.51 116.84) (layer F.SilkS) (width 0.2))
 (gr_line (start 142.24 114.3) (end 143.51 114.3) (layer F.SilkS) (width 0.2))
 (gr_line (start 142.24 116.84) (end 142.24 114.3) (layer F.SilkS) (width 0.2))
 (gr_line (start 146.05 114.3) (end 146.05 116.84) (layer F.SilkS) (width 0.2))
 (gr_line (start 144.78 114.3) (end 146.05 114.3) (layer F.SilkS) (width 0.2))
 (gr_line (start 144.78 116.84) (end 144.78 114.3) (layer F.SilkS) (width 0.2))
 (gr_line (start 148.59 114.3) (end 148.59 116.84) (layer F.SilkS) (width 0.2))
 (gr_line (start 147.32 114.3) (end 148.59 114.3) (layer F.SilkS) (width 0.2))
 (gr_line (start 147.32 116.84) (end 147.32 114.3) (layer F.SilkS) (width 0.2))
 (gr_line (start 151.13 114.3) (end 151.13 116.84) (layer F.SilkS) (width 0.2))
 (gr_line (start 149.86 114.3) (end 151.13 114.3) (layer F.SilkS) (width 0.2))
 (gr_line (start 149.86 116.84) (end 149.86 114.3) (layer F.SilkS) (width 0.2))
 (gr_line (start 153.67 114.3) (end 153.67 116.84) (layer F.SilkS) (width 0.2))
 (gr_line (start 152.4 114.3) (end 153.67 114.3) (layer F.SilkS) (width 0.2))
 (gr_line (start 152.4 116.84) (end 152.4 114.3) (layer F.SilkS) (width 0.2))
 (gr_line (start 153.67 107.95) (end 153.67 105.41) (layer F.SilkS) (width 0.2))
 (gr_line (start 152.4 107.95) (end 153.67 107.95) (layer F.SilkS) (width 0.2))
 (gr_line (start 152.4 105.41) (end 152.4 107.95) (layer F.SilkS) (width 0.2))
 (gr_line (start 151.13 107.95) (end 151.13 105.41) (layer F.SilkS) (width 0.2))
 (gr_line (start 149.86 107.95) (end 151.13 107.95) (layer F.SilkS) (width 0.2))
 (gr_line (start 149.86 105.41) (end 149.86 107.95) (layer F.SilkS) (width 0.2))
 (gr_line (start 148.59 107.95) (end 148.59 105.41) (layer F.SilkS) (width 0.2))
 (gr_line (start 147.32 107.95) (end 148.59 107.95) (layer F.SilkS) (width 0.2))
 (gr_line (start 147.32 105.41) (end 147.32 107.95) (layer F.SilkS) (width 0.2))
 (gr_line (start 146.05 107.95) (end 146.05 105.41) (layer F.SilkS) (width 0.2))
 (gr_line (start 144.78 107.95) (end 146.05 107.95) (layer F.SilkS) (width 0.2))
 (gr_line (start 144.78 105.41) (end 144.78 107.95) (layer F.SilkS) (width 0.2))
 (gr_line (start 143.51 105.41) (end 143.51 107.95) (layer F.SilkS) (width 0.2))
 (gr_line (start 142.24 107.95) (end 143.51 107.95) (layer F.SilkS) (width 0.2))
 (gr_line (start 142.24 105.41) (end 142.24 107.95) (layer F.SilkS) (width 0.2))
 (gr_line (start 156.21 116.84) (end 140.97 116.84) (layer F.SilkS) (width 0.2))
 (gr_line (start 156.21 105.41) (end 156.21 116.84) (layer F.SilkS) (width 0.2))
 (gr_line (start 140.97 105.41) (end 156.21 105.41) (layer F.SilkS) (width 0.2))
 (gr_line (start 140.97 105.41) (end 140.97 116.84) (layer F.SilkS) (width 0.2))
 (segment (start 133.985 109.76) (end 135.985 109.76) (width 0.25) (layer F.Cu) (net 1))
 (segment (start 135.985 109.76) (end 138.43 107.315) (width 0.25) (layer F.Cu) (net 1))
 (segment (start 133.985 109.76) (end 129.445 109.76) (width 0.25) (layer F.Cu) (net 1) (status 10))
 (segment (start 129.445 109.76) (end 127 107.315) (width 0.25) (layer F.Cu) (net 1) (status 20))
 (segment (start 133.985 109.61) (end 133.985 109.76) (width 0.25) (layer F.Cu) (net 1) (status 30))
 (segment (start 133.985 113.76) (end 130.945 113.76) (width 0.25) (layer F.Cu) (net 2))
 (segment (start 130.945 113.76) (end 127 109.815) (width 0.25) (layer F.Cu) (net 2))
 (segment (start 133.985 113.76) (end 133.985 113.61) (width 0.25) (layer F.Cu) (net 2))
 (segment (start 133.985 113.61) (end 137.74 109.855) (width 0.25) (layer F.Cu) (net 2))
 (segment (start 137.74 109.855) (end 138.43 109.855) (width 0.25) (layer F.Cu) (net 2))
 (segment (start 127.874999 115.689999) (end 136.47292 115.689999) (width 0.25) (layer F.Cu) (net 4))
 (segment (start 136.47292 115.689999) (end 137.227919 114.935) (width 0.25) (layer F.Cu) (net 4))
 (segment (start 137.227919 114.935) (end 138.43 114.935) (width 0.25) (layer F.Cu) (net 4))
 (segment (start 137.862919 114.935) (end 139.065 114.935) (width 0.25) (layer F.Cu) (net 4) (status 20))
 (segment (start 127.874999 115.689999) (end 127 114.815) (width 0.25) (layer F.Cu) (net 4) (status 20))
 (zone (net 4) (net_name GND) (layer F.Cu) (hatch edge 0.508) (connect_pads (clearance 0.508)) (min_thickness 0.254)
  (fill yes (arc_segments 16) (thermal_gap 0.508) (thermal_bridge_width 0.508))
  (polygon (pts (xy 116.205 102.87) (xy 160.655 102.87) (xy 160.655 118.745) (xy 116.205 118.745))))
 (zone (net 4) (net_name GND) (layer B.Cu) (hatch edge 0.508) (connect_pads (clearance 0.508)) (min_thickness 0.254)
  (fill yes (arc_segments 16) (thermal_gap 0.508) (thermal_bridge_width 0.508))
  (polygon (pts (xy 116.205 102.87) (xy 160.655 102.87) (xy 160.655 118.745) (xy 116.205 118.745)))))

